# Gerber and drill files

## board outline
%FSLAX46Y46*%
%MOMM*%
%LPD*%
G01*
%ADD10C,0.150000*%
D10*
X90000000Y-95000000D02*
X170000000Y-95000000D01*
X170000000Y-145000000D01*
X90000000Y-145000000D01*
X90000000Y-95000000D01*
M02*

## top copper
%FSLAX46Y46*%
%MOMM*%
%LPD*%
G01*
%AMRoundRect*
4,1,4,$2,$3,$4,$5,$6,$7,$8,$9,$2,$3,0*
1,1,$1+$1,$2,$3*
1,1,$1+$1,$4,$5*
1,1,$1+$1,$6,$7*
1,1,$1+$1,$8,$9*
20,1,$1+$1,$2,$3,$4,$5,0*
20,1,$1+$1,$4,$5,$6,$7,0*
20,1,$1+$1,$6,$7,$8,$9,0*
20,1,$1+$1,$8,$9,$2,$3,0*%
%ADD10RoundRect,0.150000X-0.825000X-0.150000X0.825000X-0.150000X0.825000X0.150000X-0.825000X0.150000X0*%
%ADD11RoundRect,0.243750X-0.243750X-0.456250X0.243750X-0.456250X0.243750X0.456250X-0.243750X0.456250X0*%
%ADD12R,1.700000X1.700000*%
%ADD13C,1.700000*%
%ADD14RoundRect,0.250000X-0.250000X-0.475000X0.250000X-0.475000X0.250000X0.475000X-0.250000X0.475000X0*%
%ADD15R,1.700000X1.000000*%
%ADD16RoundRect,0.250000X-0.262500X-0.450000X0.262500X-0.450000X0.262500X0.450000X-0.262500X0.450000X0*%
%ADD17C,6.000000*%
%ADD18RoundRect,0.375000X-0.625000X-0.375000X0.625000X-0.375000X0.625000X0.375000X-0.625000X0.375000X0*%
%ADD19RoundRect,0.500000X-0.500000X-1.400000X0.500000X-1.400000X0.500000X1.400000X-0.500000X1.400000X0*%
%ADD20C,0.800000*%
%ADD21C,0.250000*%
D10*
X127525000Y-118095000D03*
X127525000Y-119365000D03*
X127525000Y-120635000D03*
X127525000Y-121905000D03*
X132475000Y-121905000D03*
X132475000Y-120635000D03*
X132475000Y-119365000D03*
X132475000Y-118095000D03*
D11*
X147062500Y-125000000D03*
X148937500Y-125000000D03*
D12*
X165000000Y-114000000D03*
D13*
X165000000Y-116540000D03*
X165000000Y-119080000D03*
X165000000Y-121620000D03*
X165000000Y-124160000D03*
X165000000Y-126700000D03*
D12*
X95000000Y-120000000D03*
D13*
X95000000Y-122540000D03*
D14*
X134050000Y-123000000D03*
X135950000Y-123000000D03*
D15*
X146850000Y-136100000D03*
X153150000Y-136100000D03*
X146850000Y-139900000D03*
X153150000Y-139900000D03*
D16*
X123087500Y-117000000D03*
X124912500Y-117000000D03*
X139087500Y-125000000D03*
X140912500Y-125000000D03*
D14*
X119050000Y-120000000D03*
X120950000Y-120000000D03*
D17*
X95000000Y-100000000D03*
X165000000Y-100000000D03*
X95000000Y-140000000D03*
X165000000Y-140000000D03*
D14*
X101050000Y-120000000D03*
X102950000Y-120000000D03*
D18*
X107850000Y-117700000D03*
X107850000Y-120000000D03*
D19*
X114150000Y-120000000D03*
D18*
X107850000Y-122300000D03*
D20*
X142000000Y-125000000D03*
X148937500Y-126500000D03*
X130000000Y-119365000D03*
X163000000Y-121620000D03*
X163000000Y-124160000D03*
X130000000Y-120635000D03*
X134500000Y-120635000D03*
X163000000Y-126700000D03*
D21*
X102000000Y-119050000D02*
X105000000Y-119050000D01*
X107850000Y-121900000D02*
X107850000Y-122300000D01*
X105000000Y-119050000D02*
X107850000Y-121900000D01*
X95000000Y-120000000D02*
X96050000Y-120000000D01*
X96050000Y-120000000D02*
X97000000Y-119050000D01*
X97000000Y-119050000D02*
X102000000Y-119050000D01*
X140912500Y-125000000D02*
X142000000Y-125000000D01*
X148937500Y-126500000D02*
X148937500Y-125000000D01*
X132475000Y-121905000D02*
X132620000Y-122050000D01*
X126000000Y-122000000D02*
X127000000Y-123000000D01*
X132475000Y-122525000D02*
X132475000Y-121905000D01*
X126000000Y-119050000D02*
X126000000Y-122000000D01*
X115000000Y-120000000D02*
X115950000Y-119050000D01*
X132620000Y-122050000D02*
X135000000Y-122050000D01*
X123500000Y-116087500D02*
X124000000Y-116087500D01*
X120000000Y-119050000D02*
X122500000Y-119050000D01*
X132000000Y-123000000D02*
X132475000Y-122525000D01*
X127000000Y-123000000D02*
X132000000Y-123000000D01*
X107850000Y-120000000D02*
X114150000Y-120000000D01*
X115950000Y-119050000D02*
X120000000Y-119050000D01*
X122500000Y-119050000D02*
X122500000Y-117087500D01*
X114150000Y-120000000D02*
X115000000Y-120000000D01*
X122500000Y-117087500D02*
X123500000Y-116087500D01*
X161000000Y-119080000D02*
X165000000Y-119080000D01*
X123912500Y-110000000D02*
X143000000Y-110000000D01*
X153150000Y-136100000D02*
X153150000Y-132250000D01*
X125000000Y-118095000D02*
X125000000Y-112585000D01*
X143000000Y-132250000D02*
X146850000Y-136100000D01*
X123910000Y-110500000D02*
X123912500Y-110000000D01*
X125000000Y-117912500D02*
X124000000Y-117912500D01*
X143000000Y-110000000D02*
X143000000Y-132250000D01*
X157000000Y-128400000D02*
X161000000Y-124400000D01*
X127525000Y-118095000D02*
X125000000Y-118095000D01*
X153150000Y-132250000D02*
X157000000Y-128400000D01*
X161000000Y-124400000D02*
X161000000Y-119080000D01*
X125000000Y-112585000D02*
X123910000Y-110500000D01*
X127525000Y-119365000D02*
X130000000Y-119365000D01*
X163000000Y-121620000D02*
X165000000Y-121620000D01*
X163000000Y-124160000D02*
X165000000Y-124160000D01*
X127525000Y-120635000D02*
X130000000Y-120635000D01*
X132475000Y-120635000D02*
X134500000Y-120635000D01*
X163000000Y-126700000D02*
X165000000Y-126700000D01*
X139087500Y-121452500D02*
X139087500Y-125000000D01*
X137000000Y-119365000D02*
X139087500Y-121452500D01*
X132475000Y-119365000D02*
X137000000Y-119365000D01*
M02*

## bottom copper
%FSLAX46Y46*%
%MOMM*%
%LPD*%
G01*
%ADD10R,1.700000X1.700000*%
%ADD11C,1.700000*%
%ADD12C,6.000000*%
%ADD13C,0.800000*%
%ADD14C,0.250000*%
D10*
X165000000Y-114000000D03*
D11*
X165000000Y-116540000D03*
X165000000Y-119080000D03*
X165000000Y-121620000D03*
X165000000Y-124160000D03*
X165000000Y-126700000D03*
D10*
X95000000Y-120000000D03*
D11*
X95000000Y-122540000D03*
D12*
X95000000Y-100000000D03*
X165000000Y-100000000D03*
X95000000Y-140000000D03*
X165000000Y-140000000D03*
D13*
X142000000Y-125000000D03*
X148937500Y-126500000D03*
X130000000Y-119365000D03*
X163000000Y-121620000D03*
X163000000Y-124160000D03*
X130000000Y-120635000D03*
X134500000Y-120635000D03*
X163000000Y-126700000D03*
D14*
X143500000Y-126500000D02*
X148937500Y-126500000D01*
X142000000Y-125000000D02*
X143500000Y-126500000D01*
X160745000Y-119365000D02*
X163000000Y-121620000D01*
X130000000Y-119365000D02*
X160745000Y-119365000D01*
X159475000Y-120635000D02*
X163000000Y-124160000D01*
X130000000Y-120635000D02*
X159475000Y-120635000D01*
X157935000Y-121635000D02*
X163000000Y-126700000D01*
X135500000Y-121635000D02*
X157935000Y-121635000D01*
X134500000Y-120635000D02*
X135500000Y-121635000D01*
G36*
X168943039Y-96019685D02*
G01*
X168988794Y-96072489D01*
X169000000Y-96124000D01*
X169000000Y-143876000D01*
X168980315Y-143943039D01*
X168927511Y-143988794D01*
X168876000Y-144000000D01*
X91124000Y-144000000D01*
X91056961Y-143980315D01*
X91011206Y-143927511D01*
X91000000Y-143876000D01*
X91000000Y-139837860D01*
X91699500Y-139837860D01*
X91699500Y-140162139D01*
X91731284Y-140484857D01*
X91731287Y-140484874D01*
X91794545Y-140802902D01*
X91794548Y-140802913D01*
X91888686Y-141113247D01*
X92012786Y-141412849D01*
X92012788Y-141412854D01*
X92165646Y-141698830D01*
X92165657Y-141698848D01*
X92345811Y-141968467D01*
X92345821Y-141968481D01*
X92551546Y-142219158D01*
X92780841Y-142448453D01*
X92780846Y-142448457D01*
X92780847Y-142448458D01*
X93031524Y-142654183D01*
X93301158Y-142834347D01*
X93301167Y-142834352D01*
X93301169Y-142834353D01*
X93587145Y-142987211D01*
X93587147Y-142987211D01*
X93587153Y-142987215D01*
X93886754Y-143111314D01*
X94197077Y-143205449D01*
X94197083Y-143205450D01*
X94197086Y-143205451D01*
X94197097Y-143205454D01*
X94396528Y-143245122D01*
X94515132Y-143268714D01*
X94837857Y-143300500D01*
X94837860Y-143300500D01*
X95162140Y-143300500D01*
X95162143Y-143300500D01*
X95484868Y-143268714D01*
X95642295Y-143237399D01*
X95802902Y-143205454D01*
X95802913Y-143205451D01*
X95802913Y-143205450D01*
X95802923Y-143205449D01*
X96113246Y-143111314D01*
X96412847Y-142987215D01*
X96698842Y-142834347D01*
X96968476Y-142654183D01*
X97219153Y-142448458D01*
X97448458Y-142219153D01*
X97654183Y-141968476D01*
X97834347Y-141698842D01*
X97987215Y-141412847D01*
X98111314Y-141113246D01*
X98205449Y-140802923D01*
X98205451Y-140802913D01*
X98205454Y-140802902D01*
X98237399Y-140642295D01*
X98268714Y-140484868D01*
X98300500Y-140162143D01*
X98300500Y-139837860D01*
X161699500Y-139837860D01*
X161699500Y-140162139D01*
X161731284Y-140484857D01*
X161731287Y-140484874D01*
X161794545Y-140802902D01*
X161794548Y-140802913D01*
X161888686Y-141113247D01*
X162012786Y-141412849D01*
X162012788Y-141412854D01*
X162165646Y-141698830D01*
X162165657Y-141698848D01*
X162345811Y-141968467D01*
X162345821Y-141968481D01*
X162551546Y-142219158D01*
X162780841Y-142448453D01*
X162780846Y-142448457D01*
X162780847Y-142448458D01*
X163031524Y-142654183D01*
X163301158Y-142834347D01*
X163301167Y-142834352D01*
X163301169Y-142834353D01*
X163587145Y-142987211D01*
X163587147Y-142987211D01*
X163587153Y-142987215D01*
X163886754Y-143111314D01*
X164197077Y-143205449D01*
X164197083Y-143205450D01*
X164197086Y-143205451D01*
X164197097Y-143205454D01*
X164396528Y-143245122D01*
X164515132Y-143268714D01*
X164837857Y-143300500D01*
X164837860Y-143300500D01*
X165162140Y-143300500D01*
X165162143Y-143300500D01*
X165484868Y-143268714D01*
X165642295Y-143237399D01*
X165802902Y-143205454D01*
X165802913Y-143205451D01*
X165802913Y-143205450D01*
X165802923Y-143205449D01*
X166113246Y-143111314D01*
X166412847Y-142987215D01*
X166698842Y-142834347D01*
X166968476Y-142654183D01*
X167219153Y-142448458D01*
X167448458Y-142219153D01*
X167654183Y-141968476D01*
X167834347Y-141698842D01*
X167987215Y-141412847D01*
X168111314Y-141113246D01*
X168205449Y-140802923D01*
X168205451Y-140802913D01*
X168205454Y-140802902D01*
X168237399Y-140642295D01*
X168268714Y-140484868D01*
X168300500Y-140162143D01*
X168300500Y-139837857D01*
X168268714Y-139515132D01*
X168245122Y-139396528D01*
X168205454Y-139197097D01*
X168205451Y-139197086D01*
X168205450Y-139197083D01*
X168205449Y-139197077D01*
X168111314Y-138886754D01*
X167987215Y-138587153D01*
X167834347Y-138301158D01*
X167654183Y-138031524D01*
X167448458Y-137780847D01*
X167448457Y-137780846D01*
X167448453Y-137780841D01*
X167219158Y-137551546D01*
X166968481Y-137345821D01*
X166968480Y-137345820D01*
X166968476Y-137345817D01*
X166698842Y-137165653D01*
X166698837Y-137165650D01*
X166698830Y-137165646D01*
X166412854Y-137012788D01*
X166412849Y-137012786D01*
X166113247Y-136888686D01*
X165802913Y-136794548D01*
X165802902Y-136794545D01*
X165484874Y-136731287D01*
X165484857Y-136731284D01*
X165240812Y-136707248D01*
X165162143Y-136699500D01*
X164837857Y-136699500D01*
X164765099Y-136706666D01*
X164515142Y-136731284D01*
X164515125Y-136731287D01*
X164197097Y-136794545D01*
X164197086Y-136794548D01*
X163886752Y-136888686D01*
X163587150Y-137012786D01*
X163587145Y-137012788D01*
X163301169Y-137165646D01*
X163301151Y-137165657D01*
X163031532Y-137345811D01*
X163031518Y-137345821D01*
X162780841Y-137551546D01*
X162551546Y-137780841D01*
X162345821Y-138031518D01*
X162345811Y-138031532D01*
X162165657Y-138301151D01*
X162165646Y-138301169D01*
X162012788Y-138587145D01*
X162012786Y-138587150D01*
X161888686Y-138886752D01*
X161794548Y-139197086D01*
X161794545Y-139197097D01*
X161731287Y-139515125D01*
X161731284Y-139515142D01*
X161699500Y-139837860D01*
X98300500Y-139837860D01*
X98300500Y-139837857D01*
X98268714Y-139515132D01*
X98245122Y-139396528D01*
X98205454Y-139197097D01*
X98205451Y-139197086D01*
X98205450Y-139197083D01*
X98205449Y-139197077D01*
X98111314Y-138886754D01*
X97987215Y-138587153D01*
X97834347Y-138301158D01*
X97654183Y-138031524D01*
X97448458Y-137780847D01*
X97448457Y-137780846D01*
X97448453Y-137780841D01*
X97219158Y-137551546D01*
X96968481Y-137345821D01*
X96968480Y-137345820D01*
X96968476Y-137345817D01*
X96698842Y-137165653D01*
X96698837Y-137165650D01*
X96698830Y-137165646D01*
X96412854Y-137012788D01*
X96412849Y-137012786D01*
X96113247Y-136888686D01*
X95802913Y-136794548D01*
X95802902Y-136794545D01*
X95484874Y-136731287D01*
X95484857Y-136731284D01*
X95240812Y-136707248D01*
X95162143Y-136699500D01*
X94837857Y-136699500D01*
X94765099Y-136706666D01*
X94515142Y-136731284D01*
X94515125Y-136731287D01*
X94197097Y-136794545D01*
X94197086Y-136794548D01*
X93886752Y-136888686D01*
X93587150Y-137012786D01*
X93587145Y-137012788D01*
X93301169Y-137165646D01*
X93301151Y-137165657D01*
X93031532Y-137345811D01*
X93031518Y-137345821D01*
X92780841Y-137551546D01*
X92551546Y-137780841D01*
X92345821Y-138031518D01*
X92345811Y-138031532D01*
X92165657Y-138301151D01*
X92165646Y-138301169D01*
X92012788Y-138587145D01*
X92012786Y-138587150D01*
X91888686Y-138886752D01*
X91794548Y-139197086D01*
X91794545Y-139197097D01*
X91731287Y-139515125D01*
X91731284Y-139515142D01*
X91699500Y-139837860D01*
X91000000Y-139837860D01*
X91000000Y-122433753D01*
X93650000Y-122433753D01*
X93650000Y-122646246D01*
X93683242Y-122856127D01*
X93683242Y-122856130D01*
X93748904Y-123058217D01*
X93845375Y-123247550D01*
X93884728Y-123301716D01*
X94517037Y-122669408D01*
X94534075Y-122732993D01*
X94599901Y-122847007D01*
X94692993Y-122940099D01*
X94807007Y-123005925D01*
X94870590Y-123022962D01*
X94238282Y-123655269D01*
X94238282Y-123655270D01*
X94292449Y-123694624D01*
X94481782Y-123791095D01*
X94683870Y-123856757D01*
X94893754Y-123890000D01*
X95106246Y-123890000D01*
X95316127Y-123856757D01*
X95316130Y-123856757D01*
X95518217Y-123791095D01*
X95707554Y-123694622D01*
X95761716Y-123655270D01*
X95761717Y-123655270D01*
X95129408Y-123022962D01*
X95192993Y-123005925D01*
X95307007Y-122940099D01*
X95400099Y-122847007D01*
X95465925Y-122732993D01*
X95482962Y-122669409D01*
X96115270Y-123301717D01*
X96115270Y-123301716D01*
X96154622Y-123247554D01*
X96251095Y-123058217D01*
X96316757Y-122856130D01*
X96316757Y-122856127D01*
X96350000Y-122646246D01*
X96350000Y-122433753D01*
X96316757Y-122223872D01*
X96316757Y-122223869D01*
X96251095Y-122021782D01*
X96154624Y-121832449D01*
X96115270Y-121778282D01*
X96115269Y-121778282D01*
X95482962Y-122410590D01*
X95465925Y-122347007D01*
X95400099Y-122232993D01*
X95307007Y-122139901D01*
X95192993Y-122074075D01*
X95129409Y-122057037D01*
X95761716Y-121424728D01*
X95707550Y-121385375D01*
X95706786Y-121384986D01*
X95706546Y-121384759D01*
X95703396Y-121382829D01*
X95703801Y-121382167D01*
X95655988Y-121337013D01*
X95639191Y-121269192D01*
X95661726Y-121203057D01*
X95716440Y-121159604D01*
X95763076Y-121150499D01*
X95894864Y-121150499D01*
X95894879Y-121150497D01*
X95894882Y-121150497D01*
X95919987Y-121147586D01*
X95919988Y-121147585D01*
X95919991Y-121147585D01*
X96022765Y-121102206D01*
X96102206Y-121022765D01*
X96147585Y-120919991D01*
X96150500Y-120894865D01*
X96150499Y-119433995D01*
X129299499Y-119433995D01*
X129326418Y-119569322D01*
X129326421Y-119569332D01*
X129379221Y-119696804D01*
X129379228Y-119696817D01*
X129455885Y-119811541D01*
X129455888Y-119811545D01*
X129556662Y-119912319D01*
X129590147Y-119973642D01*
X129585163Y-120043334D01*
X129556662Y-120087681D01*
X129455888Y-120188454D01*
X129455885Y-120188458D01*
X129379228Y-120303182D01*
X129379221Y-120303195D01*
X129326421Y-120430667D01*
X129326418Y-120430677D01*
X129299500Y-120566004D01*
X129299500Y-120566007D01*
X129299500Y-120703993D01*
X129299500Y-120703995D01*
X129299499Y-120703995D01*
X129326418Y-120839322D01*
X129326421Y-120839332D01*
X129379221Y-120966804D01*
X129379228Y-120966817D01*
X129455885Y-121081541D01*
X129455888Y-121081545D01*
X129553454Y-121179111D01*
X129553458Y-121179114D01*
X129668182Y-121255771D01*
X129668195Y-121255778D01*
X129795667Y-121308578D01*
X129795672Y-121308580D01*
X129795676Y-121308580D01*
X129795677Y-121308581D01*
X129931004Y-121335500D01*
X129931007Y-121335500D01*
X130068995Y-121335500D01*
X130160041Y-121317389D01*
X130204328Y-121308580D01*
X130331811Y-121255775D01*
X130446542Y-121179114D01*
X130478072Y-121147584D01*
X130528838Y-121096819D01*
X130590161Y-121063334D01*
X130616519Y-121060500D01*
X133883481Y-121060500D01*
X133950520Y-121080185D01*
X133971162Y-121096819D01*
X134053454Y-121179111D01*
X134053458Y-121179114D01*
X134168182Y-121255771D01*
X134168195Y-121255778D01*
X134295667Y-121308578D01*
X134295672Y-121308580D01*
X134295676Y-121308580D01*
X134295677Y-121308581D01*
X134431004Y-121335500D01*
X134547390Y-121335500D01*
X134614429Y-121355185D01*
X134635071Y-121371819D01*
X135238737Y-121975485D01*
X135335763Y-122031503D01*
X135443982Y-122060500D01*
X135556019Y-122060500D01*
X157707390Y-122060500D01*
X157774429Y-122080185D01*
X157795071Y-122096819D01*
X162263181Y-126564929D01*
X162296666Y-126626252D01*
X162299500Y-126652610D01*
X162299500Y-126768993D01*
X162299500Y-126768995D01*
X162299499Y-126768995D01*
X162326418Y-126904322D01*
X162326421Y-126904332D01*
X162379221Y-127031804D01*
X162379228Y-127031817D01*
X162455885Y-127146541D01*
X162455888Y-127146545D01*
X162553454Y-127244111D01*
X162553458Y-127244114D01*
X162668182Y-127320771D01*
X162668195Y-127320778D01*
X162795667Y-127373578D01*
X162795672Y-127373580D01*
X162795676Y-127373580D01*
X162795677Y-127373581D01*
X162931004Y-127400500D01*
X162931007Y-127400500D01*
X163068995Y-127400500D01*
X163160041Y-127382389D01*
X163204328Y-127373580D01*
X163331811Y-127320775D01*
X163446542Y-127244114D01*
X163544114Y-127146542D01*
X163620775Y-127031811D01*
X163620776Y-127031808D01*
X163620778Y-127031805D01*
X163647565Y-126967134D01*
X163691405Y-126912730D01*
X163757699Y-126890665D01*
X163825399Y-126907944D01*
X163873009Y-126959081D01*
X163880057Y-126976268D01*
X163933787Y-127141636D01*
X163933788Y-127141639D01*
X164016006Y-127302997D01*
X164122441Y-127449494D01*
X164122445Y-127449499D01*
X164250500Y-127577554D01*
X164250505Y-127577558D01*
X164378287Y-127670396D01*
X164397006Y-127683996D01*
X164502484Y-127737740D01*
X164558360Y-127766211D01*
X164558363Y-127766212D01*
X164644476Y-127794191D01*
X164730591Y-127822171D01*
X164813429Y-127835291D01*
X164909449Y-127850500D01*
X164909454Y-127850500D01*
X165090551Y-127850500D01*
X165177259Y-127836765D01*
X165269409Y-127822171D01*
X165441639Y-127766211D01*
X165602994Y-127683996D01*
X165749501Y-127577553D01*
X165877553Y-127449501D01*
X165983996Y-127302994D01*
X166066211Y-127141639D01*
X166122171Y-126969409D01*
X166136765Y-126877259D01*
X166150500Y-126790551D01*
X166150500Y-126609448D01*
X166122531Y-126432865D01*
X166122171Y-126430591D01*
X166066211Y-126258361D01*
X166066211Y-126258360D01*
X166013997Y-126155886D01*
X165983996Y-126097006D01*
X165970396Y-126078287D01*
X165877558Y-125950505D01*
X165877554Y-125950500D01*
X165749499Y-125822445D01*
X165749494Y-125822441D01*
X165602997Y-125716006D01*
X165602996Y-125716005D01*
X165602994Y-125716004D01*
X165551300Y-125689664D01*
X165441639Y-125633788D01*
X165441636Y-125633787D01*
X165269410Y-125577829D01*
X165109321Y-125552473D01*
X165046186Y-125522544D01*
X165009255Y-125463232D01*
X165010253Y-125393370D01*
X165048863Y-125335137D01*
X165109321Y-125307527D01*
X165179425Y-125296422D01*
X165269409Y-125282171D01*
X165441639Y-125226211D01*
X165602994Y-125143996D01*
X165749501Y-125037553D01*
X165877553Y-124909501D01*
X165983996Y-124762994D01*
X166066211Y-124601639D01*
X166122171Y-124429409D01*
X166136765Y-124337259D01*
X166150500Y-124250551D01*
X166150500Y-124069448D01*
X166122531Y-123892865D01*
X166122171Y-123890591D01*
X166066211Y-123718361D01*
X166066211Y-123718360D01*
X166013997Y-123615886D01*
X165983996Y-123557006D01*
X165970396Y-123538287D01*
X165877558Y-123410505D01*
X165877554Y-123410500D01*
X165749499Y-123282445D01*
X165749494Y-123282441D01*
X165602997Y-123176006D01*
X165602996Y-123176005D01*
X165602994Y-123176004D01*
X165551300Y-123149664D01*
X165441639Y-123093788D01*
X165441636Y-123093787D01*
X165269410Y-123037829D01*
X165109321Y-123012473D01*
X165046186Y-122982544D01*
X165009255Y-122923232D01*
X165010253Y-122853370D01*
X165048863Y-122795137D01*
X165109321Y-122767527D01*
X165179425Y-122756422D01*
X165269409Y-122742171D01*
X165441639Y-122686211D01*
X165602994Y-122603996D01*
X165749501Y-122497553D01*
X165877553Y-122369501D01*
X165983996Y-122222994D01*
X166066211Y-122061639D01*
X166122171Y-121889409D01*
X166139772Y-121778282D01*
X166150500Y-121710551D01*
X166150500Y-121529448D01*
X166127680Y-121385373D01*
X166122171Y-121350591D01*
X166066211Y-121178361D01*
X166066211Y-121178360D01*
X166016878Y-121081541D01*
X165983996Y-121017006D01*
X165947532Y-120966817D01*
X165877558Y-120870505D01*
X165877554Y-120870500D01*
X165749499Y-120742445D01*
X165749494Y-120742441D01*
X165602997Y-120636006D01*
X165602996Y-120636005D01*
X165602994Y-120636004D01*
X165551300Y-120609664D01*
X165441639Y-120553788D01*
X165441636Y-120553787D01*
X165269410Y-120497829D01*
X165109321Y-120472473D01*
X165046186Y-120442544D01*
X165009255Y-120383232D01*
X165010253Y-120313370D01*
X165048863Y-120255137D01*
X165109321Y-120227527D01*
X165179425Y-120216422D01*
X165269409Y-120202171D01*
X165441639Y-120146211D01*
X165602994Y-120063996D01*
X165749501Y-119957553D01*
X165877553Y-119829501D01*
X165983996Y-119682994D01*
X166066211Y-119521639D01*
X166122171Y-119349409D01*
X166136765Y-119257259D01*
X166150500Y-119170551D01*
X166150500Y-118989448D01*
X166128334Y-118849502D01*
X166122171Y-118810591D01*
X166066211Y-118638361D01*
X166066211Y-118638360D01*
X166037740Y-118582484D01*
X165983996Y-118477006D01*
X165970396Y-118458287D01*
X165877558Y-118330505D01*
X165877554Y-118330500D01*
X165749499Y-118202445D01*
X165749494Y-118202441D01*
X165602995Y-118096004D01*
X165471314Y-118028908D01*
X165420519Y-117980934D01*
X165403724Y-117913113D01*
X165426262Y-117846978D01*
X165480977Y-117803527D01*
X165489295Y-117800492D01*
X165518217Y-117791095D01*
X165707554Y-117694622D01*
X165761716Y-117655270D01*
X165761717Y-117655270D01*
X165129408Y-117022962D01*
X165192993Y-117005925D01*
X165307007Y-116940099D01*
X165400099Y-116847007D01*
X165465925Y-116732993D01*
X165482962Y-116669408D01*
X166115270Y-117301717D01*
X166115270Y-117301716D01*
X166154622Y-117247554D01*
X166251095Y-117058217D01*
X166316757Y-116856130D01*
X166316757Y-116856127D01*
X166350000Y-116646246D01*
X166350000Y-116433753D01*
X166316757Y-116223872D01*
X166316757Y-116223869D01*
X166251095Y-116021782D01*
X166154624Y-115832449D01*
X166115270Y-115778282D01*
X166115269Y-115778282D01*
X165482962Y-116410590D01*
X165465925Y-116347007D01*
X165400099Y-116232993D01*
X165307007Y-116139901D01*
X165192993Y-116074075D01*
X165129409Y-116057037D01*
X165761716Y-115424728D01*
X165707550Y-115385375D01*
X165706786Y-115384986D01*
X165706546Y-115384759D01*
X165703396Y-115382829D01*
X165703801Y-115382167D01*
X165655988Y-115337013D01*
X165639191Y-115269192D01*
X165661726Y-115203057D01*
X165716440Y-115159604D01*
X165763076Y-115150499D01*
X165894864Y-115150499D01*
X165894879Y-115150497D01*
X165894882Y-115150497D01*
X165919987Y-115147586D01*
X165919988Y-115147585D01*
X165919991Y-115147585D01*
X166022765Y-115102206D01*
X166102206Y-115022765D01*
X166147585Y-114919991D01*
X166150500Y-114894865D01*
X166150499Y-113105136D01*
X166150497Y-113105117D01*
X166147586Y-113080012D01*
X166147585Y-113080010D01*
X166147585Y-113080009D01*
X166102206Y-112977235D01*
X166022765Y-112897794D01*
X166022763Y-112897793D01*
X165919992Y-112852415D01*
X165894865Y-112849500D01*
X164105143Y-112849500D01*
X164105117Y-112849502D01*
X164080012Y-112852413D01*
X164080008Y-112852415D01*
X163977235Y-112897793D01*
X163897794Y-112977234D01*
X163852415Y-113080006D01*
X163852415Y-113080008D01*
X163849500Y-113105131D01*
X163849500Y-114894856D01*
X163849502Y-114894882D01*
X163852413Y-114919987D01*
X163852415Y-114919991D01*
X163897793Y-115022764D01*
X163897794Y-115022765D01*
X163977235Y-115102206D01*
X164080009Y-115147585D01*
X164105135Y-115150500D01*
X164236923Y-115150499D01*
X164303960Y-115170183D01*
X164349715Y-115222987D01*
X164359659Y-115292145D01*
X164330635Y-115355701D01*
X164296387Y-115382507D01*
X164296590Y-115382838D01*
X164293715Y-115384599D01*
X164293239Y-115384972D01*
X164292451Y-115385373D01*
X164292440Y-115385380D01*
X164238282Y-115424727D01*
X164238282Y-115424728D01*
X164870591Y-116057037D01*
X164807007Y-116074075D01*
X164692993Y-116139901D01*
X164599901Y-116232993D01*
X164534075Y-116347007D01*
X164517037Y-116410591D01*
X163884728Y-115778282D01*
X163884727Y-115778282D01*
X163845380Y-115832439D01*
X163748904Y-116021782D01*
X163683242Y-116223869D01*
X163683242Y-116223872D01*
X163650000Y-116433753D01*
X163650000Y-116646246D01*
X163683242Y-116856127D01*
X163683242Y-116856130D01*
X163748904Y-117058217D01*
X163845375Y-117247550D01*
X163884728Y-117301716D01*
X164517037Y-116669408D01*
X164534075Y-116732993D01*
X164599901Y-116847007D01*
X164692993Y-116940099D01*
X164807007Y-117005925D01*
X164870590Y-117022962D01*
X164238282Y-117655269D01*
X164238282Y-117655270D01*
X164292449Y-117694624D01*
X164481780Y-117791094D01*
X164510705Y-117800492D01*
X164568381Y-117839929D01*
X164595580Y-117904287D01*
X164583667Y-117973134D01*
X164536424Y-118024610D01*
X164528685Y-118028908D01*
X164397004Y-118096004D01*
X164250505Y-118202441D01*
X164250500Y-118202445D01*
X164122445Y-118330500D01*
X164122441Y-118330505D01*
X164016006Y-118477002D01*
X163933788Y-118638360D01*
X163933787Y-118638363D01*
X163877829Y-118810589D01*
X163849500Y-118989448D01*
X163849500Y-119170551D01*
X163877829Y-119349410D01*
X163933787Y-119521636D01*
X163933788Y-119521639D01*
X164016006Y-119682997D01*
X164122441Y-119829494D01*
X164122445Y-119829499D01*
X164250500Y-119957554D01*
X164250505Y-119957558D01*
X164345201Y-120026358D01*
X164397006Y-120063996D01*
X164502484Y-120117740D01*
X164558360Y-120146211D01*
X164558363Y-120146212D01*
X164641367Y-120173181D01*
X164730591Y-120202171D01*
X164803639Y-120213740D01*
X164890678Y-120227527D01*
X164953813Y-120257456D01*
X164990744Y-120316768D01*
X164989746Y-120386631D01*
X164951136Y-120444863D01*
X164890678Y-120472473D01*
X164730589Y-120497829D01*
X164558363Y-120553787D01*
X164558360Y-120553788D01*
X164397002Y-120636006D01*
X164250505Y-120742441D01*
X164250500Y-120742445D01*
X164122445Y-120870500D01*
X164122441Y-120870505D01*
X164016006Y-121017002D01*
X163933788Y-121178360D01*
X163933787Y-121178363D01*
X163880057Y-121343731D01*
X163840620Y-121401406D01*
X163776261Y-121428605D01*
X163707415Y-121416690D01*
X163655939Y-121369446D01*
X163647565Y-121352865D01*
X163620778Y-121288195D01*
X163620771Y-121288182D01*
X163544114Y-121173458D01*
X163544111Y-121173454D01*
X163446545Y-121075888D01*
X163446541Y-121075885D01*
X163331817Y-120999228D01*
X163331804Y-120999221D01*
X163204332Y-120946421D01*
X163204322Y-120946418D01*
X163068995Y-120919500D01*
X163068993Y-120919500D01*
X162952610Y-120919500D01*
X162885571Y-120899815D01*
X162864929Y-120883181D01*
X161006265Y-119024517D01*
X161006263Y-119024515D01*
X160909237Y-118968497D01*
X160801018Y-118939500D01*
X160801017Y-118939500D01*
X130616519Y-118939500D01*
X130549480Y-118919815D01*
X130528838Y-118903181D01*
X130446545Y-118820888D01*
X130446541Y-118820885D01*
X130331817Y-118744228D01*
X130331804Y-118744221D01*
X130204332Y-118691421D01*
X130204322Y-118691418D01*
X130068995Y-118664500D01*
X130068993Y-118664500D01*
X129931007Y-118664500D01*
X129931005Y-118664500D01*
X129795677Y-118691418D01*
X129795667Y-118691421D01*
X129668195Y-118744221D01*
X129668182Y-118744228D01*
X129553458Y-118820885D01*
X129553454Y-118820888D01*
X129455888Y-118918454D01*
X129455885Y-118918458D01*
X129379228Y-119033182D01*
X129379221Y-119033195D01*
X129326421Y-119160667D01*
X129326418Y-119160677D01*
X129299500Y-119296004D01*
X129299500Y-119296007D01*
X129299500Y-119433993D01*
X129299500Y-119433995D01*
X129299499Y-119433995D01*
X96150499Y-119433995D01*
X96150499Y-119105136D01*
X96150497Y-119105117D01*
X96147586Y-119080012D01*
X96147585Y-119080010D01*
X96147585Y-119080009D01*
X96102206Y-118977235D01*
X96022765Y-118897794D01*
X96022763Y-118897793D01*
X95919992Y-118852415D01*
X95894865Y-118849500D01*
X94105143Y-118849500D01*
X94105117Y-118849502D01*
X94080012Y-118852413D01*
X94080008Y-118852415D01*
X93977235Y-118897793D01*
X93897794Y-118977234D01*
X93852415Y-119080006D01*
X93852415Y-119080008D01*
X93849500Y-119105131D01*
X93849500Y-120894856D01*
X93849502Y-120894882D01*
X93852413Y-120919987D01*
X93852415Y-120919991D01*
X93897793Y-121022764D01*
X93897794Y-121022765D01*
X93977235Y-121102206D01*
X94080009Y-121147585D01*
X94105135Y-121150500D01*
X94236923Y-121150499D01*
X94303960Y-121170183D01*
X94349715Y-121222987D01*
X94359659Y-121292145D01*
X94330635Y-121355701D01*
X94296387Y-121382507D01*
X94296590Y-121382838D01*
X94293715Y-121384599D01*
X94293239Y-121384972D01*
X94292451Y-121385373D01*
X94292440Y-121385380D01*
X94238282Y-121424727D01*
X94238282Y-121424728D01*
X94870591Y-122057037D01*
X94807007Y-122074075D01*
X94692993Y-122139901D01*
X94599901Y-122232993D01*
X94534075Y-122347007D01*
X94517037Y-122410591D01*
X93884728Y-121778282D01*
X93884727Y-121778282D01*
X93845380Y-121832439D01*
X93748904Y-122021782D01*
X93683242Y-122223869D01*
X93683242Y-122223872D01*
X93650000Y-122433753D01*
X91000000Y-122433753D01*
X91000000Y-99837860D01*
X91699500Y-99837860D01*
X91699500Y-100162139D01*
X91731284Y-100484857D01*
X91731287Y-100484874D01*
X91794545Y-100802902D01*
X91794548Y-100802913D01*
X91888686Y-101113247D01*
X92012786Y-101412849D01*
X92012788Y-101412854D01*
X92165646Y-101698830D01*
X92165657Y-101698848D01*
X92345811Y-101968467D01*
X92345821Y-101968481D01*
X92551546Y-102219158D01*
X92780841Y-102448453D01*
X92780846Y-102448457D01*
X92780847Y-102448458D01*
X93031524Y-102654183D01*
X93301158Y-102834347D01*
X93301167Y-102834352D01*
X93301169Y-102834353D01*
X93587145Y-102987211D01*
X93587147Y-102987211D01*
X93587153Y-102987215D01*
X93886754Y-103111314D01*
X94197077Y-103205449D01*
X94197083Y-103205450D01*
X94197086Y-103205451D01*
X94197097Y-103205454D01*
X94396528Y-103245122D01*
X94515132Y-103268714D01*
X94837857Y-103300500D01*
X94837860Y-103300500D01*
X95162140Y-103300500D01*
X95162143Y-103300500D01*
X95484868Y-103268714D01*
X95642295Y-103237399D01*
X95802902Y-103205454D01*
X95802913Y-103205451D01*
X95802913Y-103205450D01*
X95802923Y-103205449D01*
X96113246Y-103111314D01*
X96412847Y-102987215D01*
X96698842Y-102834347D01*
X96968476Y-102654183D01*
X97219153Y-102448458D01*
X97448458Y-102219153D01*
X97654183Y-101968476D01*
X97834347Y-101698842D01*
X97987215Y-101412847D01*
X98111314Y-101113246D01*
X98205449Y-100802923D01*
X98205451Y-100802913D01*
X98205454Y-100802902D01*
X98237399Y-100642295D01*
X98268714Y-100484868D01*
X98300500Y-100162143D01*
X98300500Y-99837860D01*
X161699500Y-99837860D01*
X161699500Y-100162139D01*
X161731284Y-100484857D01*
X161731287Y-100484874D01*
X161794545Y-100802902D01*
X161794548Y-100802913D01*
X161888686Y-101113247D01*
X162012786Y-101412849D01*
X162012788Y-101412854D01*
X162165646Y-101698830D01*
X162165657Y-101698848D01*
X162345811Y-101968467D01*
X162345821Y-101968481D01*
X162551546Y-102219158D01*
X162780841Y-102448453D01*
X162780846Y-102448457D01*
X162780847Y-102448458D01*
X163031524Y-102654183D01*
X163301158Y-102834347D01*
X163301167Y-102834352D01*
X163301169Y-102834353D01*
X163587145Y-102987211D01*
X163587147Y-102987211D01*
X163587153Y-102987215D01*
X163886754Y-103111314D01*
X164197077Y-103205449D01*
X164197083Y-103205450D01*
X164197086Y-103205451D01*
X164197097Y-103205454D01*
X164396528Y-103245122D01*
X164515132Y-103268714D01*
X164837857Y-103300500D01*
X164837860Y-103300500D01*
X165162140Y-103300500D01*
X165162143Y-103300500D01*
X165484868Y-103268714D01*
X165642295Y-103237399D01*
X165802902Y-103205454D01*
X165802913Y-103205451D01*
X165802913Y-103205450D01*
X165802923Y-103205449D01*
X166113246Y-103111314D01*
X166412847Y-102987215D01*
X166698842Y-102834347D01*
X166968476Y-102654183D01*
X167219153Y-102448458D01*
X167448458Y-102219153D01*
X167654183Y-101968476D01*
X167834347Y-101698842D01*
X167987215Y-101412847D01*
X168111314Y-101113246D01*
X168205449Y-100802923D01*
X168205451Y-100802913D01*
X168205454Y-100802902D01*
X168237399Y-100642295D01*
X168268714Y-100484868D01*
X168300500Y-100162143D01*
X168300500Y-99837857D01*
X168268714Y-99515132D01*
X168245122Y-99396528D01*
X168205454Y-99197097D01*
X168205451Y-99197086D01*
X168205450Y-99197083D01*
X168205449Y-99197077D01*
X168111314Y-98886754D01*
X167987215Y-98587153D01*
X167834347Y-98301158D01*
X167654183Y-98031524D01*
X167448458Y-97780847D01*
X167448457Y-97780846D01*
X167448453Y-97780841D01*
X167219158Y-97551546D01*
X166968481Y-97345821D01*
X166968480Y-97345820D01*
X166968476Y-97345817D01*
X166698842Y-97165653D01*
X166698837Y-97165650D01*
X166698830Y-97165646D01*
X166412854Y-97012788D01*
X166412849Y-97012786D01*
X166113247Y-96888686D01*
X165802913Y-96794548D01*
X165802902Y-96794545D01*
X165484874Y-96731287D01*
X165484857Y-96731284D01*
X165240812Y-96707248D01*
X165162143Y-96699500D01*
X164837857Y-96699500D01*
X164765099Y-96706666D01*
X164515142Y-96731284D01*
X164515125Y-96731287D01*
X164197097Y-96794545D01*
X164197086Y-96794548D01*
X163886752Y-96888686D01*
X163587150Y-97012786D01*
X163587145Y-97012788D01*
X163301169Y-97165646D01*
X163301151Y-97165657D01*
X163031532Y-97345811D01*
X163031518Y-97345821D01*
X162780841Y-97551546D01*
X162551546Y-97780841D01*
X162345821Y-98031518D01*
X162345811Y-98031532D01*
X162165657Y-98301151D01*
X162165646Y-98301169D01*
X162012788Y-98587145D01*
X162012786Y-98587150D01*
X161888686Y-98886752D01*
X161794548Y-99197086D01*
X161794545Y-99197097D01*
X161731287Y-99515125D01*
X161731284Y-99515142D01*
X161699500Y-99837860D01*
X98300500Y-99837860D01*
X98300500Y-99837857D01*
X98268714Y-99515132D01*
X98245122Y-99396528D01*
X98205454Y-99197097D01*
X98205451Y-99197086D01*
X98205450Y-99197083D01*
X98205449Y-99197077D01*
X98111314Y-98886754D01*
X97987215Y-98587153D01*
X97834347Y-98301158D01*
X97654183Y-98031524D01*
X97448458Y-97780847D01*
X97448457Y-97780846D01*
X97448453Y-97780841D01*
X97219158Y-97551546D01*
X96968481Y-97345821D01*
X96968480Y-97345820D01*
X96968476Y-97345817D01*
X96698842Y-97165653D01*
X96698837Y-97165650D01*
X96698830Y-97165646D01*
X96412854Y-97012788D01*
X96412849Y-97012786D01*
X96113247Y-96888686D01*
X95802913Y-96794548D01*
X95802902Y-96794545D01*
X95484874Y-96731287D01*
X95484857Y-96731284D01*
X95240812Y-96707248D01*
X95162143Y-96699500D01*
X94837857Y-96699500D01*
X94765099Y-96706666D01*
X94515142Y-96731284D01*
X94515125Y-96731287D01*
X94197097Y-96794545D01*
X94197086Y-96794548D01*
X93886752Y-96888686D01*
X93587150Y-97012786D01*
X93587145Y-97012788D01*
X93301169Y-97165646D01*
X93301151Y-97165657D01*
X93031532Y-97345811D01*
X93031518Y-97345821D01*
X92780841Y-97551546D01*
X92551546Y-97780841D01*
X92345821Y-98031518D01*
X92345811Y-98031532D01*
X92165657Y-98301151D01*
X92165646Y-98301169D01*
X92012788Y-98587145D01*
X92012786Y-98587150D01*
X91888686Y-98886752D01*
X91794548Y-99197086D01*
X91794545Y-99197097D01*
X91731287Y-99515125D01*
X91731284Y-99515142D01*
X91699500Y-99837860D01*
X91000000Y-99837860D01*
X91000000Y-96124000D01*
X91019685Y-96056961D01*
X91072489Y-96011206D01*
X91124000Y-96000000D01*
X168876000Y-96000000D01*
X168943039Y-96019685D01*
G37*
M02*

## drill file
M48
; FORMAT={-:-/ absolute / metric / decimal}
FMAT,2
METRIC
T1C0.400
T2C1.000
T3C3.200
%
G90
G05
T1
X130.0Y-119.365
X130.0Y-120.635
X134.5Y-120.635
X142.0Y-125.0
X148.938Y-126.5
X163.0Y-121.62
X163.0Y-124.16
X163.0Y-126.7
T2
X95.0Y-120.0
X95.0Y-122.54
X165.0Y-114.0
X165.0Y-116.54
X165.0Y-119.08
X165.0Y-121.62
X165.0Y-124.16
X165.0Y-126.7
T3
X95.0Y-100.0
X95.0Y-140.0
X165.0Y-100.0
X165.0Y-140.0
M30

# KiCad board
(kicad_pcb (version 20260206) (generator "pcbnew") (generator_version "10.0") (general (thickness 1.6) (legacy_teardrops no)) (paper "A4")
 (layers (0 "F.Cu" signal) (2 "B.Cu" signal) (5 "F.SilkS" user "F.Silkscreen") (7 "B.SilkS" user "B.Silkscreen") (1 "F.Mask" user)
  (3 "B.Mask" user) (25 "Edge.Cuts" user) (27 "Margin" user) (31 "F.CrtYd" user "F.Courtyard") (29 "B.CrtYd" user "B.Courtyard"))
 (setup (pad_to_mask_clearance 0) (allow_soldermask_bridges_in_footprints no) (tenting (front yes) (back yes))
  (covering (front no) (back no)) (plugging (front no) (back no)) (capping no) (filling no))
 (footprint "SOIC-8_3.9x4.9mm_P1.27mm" (layer "F.Cu") (at 130 120)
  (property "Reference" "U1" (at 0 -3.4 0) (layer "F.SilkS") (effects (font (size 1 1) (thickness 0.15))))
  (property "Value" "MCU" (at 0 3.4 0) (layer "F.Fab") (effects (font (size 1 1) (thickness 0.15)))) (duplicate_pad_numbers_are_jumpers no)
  (pad "1" smd roundrect (at -2.475 -1.905) (size 1.95 0.6) (layers "F.Cu" "F.Mask" "F.Paste") (roundrect_rratio 0.25) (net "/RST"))
  (pad "2" smd roundrect (at -2.475 -0.635) (size 1.95 0.6) (layers "F.Cu" "F.Mask" "F.Paste") (roundrect_rratio 0.25) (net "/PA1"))
  (pad "3" smd roundrect (at -2.475 0.635) (size 1.95 0.6) (layers "F.Cu" "F.Mask" "F.Paste") (roundrect_rratio 0.25) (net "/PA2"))
  (pad "4" smd roundrect (at -2.475 1.905) (size 1.95 0.6) (layers "F.Cu" "F.Mask" "F.Paste") (roundrect_rratio 0.25) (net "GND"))
  (pad "5" smd roundrect (at 2.475 1.905) (size 1.95 0.6) (layers "F.Cu" "F.Mask" "F.Paste") (roundrect_rratio 0.25) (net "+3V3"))
  (pad "6" smd roundrect (at 2.475 0.635) (size 1.95 0.6) (layers "F.Cu" "F.Mask" "F.Paste") (roundrect_rratio 0.25) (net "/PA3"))
  (pad "7" smd roundrect (at 2.475 -0.635) (size 1.95 0.6) (layers "F.Cu" "F.Mask" "F.Paste") (roundrect_rratio 0.25) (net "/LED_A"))
  (pad "8" smd roundrect (at 2.475 -1.905) (size 1.95 0.6) (layers "F.Cu" "F.Mask" "F.Paste") (roundrect_rratio 0.25) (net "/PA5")))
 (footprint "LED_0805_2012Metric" (layer "F.Cu") (at 148 125)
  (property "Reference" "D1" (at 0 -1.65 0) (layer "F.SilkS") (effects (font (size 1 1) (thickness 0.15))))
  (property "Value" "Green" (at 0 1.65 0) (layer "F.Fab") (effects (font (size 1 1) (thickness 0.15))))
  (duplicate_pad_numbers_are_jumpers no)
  (pad "1" smd roundrect (at -0.9375 0) (size 0.975 1.4) (layers "F.Cu" "F.Mask" "F.Paste") (roundrect_rratio 0.25) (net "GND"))
  (pad "2" smd roundrect (at 0.9375 0) (size 0.975 1.4) (layers "F.Cu" "F.Mask" "F.Paste") (roundrect_rratio 0.25) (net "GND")))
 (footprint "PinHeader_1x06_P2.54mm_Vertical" (layer "F.Cu") (at 165 114)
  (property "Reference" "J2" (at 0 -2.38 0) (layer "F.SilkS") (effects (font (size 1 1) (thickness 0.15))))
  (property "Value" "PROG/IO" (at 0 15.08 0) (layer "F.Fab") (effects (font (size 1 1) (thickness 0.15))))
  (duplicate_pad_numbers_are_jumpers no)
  (pad "1" thru_hole rect (at 0 0) (size 1.7 1.7) (drill 1) (layers "*.Cu" "*.Mask") (remove_unused_layers no) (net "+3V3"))
  (pad "2" thru_hole circle (at 0 2.54) (size 1.7 1.7) (drill 1) (layers "*.Cu" "*.Mask") (remove_unused_layers no) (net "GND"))
  (pad "3" thru_hole circle (at 0 5.08) (size 1.7 1.7) (drill 1) (layers "*.Cu" "*.Mask") (remove_unused_layers no) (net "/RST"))
  (pad "4" thru_hole circle (at 0 7.62) (size 1.7 1.7) (drill 1) (layers "*.Cu" "*.Mask") (remove_unused_layers no) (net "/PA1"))
  (pad "5" thru_hole circle (at 0 10.16) (size 1.7 1.7) (drill 1) (layers "*.Cu" "*.Mask") (remove_unused_layers no) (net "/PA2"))
  (pad "6" thru_hole circle (at 0 12.7) (size 1.7 1.7) (drill 1) (layers "*.Cu" "*.Mask") (remove_unused_layers no) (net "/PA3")))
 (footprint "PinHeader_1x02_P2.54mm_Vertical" (layer "F.Cu") (at 95 120)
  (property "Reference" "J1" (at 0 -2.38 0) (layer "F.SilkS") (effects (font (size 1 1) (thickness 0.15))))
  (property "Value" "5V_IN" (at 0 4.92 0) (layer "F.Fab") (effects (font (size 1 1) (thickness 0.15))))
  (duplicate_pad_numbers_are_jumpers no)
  (pad "1" thru_hole rect (at 0 0) (size 1.7 1.7) (drill 1) (layers "*.Cu" "*.Mask") (remove_unused_layers no) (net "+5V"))
  (pad "2" thru_hole circle (at 0 2.54) (size 1.7 1.7) (drill 1) (layers "*.Cu" "*.Mask") (remove_unused_layers no) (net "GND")))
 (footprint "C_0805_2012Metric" (layer "F.Cu") (at 135 123)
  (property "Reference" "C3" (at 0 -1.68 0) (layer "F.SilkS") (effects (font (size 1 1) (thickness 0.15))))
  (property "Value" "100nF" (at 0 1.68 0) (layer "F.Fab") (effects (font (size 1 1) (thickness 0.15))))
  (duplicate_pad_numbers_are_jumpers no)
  (pad "1" smd roundrect (at -0.95 0) (size 1 1.45) (layers "F.Cu" "F.Mask" "F.Paste") (roundrect_rratio 0.25) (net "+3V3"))
  (pad "2" smd roundrect (at 0.95 0) (size 1 1.45) (layers "F.Cu" "F.Mask" "F.Paste") (roundrect_rratio 0.25) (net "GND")))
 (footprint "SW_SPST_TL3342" (layer "F.Cu") (at 150 138)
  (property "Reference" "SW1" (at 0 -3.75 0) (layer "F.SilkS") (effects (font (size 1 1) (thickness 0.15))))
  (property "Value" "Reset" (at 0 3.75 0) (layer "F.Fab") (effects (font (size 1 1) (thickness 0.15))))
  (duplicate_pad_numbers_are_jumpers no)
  (pad "1" smd rect (at -3.15 -1.9) (size 1.7 1) (layers "F.Cu" "F.Mask" "F.Paste") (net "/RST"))
  (pad "1" smd rect (at 3.15 -1.9) (size 1.7 1) (layers "F.Cu" "F.Mask" "F.Paste") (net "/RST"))
  (pad "2" smd rect (at -3.15 1.9) (size 1.7 1) (layers "F.Cu" "F.Mask" "F.Paste") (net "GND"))
  (pad "2" smd rect (at 3.15 1.9) (size 1.7 1) (layers "F.Cu" "F.Mask" "F.Paste") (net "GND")))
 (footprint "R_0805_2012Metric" (layer "F.Cu") (at 124 117)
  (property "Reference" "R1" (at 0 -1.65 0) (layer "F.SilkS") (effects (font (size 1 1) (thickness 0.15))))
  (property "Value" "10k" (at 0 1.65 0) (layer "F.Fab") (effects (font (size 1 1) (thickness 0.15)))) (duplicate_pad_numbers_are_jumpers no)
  (pad "1" smd roundrect (at -0.9125 0) (size 1.025 1.4) (layers "F.Cu" "F.Mask" "F.Paste") (roundrect_rratio 0.243902) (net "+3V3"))
  (pad "2" smd roundrect (at 0.9125 0) (size 1.025 1.4) (layers "F.Cu" "F.Mask" "F.Paste") (roundrect_rratio 0.243902) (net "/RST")))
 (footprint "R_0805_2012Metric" (layer "F.Cu") (at 140 125)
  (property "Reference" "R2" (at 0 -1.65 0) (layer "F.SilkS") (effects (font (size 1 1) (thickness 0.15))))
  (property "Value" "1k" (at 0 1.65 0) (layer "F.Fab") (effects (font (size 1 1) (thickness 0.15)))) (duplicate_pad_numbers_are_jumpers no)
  (pad "1" smd roundrect (at -0.9125 0) (size 1.025 1.4) (layers "F.Cu" "F.Mask" "F.Paste") (roundrect_rratio 0.243902) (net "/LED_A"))
  (pad "2" smd roundrect (at 0.9125 0) (size 1.025 1.4) (layers "F.Cu" "F.Mask" "F.Paste") (roundrect_rratio 0.243902) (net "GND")))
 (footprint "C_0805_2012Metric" (layer "F.Cu") (at 120 120)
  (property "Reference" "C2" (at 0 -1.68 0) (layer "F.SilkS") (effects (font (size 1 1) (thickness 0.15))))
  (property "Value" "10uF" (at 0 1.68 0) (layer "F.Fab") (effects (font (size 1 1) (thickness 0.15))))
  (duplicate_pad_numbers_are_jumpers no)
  (pad "1" smd roundrect (at -0.95 0) (size 1 1.45) (layers "F.Cu" "F.Mask" "F.Paste") (roundrect_rratio 0.25) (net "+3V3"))
  (pad "2" smd roundrect (at 0.95 0) (size 1 1.45) (layers "F.Cu" "F.Mask" "F.Paste") (roundrect_rratio 0.25) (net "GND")))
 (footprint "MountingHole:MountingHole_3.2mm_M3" (layer "F.Cu") (at 95 100)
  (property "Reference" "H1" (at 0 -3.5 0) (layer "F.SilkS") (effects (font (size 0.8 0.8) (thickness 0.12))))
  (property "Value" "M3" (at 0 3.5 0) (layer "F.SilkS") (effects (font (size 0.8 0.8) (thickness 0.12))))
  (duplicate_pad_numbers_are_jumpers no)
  (pad "" thru_hole circle (at 0 0) (size 6 6) (drill 3.2) (layers "*.Cu" "*.Mask") (remove_unused_layers no)))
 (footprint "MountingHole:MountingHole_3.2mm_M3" (layer "F.Cu") (at 165 100)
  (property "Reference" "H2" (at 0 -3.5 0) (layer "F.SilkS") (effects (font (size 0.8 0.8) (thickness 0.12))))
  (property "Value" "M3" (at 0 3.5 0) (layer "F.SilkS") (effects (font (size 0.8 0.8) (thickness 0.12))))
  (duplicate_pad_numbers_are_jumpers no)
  (pad "" thru_hole circle (at 0 0) (size 6 6) (drill 3.2) (layers "*.Cu" "*.Mask") (remove_unused_layers no)))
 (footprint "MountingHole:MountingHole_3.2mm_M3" (layer "F.Cu") (at 95 140)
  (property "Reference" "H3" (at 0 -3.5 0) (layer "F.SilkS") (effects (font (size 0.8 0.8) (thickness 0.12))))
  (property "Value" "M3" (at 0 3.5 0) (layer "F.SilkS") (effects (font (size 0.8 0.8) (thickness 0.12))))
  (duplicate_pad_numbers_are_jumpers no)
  (pad "" thru_hole circle (at 0 0) (size 6 6) (drill 3.2) (layers "*.Cu" "*.Mask") (remove_unused_layers no)))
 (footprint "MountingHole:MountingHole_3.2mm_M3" (layer "F.Cu") (at 165 140)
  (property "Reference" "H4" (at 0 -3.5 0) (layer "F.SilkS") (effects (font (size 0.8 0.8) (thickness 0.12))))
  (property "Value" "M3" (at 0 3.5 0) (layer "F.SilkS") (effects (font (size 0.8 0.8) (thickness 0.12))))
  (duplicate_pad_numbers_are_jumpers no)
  (pad "" thru_hole circle (at 0 0) (size 6 6) (drill 3.2) (layers "*.Cu" "*.Mask") (remove_unused_layers no)))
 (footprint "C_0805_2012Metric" (layer "F.Cu") (at 102 120)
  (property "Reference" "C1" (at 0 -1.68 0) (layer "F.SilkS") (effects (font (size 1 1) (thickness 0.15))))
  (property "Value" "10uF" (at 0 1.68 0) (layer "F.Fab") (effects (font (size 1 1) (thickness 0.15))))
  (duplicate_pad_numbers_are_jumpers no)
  (pad "1" smd roundrect (at -0.95 0) (size 1 1.45) (layers "F.Cu" "F.Mask" "F.Paste") (roundrect_rratio 0.25) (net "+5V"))
  (pad "2" smd roundrect (at 0.95 0) (size 1 1.45) (layers "F.Cu" "F.Mask" "F.Paste") (roundrect_rratio 0.25) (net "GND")))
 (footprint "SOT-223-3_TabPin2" (layer "F.Cu") (at 111 120)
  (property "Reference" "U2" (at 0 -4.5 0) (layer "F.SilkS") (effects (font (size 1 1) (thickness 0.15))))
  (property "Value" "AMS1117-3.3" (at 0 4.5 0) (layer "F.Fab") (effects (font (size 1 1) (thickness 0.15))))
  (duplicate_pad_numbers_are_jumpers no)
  (pad "1" smd roundrect (at -3.15 -2.3) (size 2 1.5) (layers "F.Cu" "F.Mask" "F.Paste") (roundrect_rratio 0.25) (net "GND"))
  (pad "2" smd roundrect (at -3.15 0) (size 2 1.5) (layers "F.Cu" "F.Mask" "F.Paste") (roundrect_rratio 0.25) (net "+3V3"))
  (pad "2" smd roundrect (at 3.15 0) (size 2 3.8) (layers "F.Cu" "F.Mask" "F.Paste") (roundrect_rratio 0.25) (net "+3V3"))
  (pad "3" smd roundrect (at -3.15 2.3) (size 2 1.5) (layers "F.Cu" "F.Mask" "F.Paste") (roundrect_rratio 0.25) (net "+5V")))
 (gr_rect (start 90 95) (end 170 145) (stroke (width 0.15) (type solid)) (fill no) (layer "Edge.Cuts"))
 (segment (start 102 119.05) (end 105 119.05) (width 0.25) (layer "F.Cu") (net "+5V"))
 (segment (start 107.85 121.9) (end 107.85 122.3) (width 0.25) (layer "F.Cu") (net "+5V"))
 (segment (start 105 119.05) (end 107.85 121.9) (width 0.25) (layer "F.Cu") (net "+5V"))
 (segment (start 95 120) (end 96.05 120) (width 0.25) (layer "F.Cu") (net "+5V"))
 (segment (start 96.05 120) (end 97 119.05) (width 0.25) (layer "F.Cu") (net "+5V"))
 (segment (start 97 119.05) (end 102 119.05) (width 0.25) (layer "F.Cu") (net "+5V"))
 (segment (start 140.9125 125) (end 142 125) (width 0.25) (layer "F.Cu") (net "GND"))
 (segment (start 148.9375 126.5) (end 148.9375 125) (width 0.25) (layer "F.Cu") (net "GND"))
 (via (at 142 125) (size 0.8) (drill 0.4) (layers "F.Cu" "B.Cu") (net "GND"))
 (via (at 148.9375 126.5) (size 0.8) (drill 0.4) (layers "F.Cu" "B.Cu") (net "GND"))
 (segment (start 143.5 126.5) (end 148.9375 126.5) (width 0.25) (layer "B.Cu") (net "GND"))
 (segment (start 142 125) (end 143.5 126.5) (width 0.25) (layer "B.Cu") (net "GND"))
 (segment (start 132.475 121.905) (end 132.62 122.05) (width 0.25) (layer "F.Cu") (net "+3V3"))
 (segment (start 126 122) (end 127 123) (width 0.25) (layer "F.Cu") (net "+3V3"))
 (segment (start 132.475 122.525) (end 132.475 121.905) (width 0.25) (layer "F.Cu") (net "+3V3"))
 (segment (start 126 119.05) (end 126 122) (width 0.25) (layer "F.Cu") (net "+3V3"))
 (segment (start 115 120) (end 115.95 119.05) (width 0.25) (layer "F.Cu") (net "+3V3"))
 (segment (start 132.62 122.05) (end 135 122.05) (width 0.25) (layer "F.Cu") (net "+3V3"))
 (segment (start 123.5 116.0875) (end 124 116.0875) (width 0.25) (layer "F.Cu") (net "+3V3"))
 (segment (start 120 119.05) (end 122.5 119.05) (width 0.25) (layer "F.Cu") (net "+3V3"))
 (segment (start 132 123) (end 132.475 122.525) (width 0.25) (layer "F.Cu") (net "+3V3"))
 (segment (start 127 123) (end 132 123) (width 0.25) (layer "F.Cu") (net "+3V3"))
 (segment (start 107.85 120) (end 114.15 120) (width 0.25) (layer "F.Cu") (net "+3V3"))
 (segment (start 115.95 119.05) (end 120 119.05) (width 0.25) (layer "F.Cu") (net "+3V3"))
 (segment (start 122.5 119.05) (end 122.5 117.0875) (width 0.25) (layer "F.Cu") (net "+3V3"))
 (segment (start 114.15 120) (end 115 120) (width 0.25) (layer "F.Cu") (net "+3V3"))
 (segment (start 122.5 117.0875) (end 123.5 116.0875) (width 0.25) (layer "F.Cu") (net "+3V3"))
 (segment (start 161 119.08) (end 165 119.08) (width 0.25) (layer "F.Cu") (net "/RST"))
 (segment (start 123.9125 110) (end 143 110) (width 0.25) (layer "F.Cu") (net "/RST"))
 (segment (start 153.15 136.1) (end 153.15 132.25) (width 0.25) (layer "F.Cu") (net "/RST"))
 (segment (start 125 118.095) (end 125 112.585) (width 0.25) (layer "F.Cu") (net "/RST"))
 (segment (start 143 132.25) (end 146.85 136.1) (width 0.25) (layer "F.Cu") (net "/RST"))
 (segment (start 123.91 110.5) (end 123.9125 110) (width 0.25) (layer "F.Cu") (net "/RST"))
 (segment (start 125 117.9125) (end 124 117.9125) (width 0.25) (layer "F.Cu") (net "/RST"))
 (segment (start 143 110) (end 143 132.25) (width 0.25) (layer "F.Cu") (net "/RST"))
 (segment (start 157 128.4) (end 161 124.4) (width 0.25) (layer "F.Cu") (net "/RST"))
 (segment (start 127.525 118.095) (end 125 118.095) (width 0.25) (layer "F.Cu") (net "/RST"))
 (segment (start 153.15 132.25) (end 157 128.4) (width 0.25) (layer "F.Cu") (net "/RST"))
 (segment (start 161 124.4) (end 161 119.08) (width 0.25) (layer "F.Cu") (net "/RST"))
 (segment (start 125 112.585) (end 123.91 110.5) (width 0.25) (layer "F.Cu") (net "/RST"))
 (segment (start 127.525 119.365) (end 130 119.365) (width 0.25) (layer "F.Cu") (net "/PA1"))
 (segment (start 163 121.62) (end 165 121.62) (width 0.25) (layer "F.Cu") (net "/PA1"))
 (via (at 130 119.365) (size 0.8) (drill 0.4) (layers "F.Cu" "B.Cu") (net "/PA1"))
 (via (at 163 121.62) (size 0.8) (drill 0.4) (layers "F.Cu" "B.Cu") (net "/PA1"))
 (segment (start 160.745 119.365) (end 163 121.62) (width 0.25) (layer "B.Cu") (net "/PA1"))
 (segment (start 130 119.365) (end 160.745 119.365) (width 0.25) (layer "B.Cu") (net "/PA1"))
 (segment (start 163 124.16) (end 165 124.16) (width 0.25) (layer "F.Cu") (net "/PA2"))
 (segment (start 127.525 120.635) (end 130 120.635) (width 0.25) (layer "F.Cu") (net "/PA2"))
 (via (at 163 124.16) (size 0.8) (drill 0.4) (layers "F.Cu" "B.Cu") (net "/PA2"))
 (via (at 130 120.635) (size 0.8) (drill 0.4) (layers "F.Cu" "B.Cu") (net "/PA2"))
 (segment (start 159.475 120.635) (end 163 124.16) (width 0.25) (layer "B.Cu") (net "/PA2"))
 (segment (start 130 120.635) (end 159.475 120.635) (width 0.25) (layer "B.Cu") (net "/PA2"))
 (segment (start 132.475 120.635) (end 134.5 120.635) (width 0.25) (layer "F.Cu") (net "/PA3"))
 (segment (start 163 126.7) (end 165 126.7) (width 0.25) (layer "F.Cu") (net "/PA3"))
 (via (at 134.5 120.635) (size 0.8) (drill 0.4) (layers "F.Cu" "B.Cu") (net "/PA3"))
 (via (at 163 126.7) (size 0.8) (drill 0.4) (layers "F.Cu" "B.Cu") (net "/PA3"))
 (segment (start 157.935 121.635) (end 163 126.7) (width 0.25) (layer "B.Cu") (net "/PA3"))
 (segment (start 135.5 121.635) (end 157.935 121.635) (width 0.25) (layer "B.Cu") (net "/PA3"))
 (segment (start 134.5 120.635) (end 135.5 121.635) (width 0.25) (layer "B.Cu") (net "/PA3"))
 (segment (start 139.0875 121.4525) (end 139.0875 125) (width 0.25) (layer "F.Cu") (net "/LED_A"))
 (segment (start 137 119.365) (end 139.0875 121.4525) (width 0.25) (layer "F.Cu") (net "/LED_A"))
 (segment (start 132.475 119.365) (end 137 119.365) (width 0.25) (layer "F.Cu") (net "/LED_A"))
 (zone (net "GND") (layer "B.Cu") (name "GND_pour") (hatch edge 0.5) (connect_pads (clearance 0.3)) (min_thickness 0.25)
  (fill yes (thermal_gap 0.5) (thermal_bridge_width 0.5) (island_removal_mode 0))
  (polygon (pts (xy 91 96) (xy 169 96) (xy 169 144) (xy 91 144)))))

